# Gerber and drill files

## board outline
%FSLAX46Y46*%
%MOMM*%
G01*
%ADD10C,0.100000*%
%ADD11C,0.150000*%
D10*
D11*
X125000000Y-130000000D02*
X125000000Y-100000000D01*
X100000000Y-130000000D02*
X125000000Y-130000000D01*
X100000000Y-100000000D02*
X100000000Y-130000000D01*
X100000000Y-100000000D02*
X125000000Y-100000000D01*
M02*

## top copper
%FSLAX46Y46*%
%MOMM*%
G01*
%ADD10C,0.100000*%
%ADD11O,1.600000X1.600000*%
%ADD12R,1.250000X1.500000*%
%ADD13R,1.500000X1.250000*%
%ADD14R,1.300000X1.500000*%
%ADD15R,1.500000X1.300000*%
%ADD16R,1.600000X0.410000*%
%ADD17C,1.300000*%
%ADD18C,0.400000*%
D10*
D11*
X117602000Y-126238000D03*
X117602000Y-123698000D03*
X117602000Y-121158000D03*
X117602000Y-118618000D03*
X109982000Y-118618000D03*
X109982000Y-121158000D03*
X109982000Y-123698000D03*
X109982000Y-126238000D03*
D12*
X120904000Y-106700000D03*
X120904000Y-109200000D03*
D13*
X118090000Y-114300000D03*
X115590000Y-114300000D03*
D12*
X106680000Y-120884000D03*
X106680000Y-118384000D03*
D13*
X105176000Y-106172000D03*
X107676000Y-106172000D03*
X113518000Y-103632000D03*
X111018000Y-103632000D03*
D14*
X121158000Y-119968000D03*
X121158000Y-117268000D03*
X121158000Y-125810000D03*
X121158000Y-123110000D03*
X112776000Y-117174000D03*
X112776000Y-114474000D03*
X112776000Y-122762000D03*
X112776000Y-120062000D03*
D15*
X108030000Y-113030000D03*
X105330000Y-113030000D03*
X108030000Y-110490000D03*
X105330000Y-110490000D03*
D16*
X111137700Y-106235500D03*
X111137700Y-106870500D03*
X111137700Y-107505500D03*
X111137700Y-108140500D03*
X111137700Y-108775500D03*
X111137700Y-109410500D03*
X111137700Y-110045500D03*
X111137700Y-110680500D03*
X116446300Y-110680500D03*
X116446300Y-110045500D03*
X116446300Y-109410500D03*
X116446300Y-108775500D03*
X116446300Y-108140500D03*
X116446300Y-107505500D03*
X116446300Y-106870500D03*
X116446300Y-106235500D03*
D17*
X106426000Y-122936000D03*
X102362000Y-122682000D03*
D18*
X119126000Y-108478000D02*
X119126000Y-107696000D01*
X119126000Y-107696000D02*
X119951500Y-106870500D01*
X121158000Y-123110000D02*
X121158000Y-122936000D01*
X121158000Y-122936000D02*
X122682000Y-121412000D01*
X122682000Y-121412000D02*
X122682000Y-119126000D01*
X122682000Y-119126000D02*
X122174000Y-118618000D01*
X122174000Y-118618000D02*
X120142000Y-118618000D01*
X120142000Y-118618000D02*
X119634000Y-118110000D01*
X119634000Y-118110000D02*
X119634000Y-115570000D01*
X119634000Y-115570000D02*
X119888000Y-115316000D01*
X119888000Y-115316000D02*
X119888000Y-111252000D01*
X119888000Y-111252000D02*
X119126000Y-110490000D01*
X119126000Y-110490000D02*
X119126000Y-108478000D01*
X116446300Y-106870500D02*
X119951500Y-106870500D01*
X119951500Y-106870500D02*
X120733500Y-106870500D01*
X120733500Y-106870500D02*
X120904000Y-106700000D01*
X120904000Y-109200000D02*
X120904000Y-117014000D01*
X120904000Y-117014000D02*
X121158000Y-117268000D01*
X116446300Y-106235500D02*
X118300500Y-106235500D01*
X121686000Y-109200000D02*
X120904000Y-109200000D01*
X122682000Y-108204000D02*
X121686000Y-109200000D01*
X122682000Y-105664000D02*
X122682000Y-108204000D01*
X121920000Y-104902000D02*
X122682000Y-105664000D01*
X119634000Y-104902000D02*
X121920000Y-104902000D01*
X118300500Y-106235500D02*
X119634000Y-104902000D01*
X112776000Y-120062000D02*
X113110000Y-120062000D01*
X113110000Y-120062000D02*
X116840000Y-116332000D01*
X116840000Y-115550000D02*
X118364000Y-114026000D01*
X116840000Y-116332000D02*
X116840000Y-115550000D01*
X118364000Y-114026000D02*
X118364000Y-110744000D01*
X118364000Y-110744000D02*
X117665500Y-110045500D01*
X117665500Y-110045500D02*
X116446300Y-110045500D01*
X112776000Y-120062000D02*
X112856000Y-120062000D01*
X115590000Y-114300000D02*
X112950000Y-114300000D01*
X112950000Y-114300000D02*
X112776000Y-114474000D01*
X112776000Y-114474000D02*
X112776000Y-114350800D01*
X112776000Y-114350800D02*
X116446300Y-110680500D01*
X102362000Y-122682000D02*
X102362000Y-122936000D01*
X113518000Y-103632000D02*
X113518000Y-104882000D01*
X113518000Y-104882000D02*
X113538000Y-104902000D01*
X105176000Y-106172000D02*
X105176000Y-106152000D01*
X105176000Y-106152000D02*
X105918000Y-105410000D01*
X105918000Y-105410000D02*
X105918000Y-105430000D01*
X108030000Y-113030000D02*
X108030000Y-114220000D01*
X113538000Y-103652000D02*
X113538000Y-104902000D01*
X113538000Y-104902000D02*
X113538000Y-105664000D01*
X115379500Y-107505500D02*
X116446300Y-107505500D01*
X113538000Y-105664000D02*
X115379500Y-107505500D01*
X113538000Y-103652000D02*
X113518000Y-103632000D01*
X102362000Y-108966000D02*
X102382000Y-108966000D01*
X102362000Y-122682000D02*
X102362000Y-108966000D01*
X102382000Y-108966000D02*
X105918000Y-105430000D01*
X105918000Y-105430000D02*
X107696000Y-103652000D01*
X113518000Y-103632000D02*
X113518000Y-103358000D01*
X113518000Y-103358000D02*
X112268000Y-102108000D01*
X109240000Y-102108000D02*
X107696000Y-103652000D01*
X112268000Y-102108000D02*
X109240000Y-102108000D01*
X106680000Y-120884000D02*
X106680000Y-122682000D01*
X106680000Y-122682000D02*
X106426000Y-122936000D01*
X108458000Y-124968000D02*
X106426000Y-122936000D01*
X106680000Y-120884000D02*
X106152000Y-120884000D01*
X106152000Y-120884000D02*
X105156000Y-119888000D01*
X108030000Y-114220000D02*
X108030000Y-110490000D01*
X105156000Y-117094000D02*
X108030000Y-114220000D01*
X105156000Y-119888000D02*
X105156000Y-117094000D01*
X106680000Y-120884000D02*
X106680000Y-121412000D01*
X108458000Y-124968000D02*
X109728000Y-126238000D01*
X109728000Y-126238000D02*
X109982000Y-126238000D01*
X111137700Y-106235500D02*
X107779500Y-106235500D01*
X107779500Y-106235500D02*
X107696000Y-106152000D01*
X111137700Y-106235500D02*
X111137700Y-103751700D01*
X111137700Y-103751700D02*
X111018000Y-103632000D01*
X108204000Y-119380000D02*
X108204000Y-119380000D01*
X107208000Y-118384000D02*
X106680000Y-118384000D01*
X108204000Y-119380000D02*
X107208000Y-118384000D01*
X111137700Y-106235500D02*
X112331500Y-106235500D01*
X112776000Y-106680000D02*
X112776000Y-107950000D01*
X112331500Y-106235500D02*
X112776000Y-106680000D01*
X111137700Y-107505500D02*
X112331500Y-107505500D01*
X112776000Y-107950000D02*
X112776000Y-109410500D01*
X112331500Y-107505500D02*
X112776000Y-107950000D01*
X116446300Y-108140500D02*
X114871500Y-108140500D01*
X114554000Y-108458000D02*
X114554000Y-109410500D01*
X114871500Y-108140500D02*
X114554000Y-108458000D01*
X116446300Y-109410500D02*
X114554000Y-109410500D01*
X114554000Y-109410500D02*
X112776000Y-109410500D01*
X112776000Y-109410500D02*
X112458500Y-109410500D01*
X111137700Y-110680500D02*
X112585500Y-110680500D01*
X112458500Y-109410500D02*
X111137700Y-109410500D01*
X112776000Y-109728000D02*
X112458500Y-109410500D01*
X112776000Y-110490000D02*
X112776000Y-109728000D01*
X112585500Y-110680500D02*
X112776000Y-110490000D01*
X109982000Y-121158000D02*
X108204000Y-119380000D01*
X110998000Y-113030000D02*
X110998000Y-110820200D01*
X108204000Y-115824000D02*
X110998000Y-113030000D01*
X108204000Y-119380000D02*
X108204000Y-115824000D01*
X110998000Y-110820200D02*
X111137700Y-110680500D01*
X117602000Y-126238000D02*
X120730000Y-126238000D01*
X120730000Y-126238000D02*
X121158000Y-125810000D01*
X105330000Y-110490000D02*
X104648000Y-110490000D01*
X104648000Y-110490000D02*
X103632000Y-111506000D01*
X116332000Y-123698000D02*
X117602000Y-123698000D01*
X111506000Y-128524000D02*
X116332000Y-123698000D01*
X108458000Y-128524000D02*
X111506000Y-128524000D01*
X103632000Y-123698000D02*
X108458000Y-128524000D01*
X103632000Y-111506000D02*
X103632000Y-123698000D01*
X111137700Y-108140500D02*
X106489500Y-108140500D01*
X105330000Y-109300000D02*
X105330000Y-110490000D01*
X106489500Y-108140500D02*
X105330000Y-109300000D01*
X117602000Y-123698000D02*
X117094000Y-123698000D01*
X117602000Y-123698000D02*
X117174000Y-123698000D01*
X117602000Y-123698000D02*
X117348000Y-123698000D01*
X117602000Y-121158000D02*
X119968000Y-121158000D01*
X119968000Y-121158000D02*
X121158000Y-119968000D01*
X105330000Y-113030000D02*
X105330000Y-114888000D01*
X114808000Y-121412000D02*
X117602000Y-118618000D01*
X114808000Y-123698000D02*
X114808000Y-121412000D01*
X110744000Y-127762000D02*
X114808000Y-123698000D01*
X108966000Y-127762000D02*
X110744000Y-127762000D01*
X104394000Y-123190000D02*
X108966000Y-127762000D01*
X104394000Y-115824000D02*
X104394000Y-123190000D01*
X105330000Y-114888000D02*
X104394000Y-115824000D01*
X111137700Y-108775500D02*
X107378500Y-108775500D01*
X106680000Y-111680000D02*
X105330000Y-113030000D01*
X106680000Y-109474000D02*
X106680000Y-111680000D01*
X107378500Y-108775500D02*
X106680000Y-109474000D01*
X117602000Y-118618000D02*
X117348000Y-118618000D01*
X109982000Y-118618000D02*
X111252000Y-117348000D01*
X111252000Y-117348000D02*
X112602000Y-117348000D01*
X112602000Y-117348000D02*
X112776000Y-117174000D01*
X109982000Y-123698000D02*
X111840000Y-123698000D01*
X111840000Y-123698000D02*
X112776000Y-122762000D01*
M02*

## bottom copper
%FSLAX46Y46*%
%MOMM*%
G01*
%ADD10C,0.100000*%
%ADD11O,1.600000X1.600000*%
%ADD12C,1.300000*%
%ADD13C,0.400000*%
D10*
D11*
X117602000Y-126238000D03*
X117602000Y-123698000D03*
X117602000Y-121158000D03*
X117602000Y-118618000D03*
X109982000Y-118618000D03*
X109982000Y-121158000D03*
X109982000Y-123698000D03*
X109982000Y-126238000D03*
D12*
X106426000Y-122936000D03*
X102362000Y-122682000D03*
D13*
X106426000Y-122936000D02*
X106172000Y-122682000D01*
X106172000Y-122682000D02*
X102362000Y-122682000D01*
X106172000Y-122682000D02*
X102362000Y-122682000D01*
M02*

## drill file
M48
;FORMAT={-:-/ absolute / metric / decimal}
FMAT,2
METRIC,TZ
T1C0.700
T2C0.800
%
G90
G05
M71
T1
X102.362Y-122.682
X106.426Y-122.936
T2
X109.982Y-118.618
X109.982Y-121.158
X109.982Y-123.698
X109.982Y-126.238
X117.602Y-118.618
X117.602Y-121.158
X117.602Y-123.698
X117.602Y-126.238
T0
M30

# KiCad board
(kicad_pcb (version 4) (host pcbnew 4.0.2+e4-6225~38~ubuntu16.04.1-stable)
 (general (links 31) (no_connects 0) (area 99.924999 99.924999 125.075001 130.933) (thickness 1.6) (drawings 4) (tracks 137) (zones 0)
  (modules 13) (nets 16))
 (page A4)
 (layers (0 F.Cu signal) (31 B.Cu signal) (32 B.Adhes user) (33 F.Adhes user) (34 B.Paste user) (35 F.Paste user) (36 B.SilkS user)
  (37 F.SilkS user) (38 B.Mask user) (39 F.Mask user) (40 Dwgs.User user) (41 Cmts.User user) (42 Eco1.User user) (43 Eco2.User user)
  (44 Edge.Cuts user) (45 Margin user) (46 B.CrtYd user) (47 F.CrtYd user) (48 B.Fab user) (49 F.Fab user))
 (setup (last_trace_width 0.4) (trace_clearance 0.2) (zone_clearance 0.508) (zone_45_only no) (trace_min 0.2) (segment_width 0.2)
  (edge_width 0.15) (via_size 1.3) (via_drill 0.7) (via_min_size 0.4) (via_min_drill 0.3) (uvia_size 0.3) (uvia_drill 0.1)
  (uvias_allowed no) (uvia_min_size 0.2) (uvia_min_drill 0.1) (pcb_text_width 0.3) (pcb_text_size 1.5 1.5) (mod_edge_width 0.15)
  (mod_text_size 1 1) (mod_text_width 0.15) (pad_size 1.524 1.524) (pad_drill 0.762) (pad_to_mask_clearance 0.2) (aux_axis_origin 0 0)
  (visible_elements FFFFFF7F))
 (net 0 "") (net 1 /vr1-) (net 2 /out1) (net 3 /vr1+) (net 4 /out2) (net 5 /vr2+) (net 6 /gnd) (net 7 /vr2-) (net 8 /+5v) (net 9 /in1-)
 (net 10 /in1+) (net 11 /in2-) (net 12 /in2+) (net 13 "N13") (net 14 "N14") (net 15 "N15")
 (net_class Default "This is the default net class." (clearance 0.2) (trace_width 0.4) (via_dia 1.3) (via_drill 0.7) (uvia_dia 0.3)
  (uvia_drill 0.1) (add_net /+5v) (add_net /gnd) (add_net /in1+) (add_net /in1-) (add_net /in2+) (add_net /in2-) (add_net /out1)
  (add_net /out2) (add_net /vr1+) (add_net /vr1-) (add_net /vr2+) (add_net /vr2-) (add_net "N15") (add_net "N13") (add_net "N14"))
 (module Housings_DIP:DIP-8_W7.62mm (layer F.Cu) (at 117.602 126.238 180)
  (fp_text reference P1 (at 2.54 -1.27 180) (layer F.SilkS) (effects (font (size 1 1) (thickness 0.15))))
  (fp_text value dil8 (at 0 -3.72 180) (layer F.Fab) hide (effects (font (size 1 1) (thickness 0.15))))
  (pad 1 thru_hole oval (at 0 0 180) (size 1.6 1.6) (drill 0.8) (layers *.Cu *.Mask F.SilkS) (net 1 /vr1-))
  (pad 2 thru_hole oval (at 0 2.54 180) (size 1.6 1.6) (drill 0.8) (layers *.Cu *.Mask F.SilkS) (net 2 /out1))
  (pad 3 thru_hole oval (at 0 5.08 180) (size 1.6 1.6) (drill 0.8) (layers *.Cu *.Mask F.SilkS) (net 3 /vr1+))
  (pad 4 thru_hole oval (at 0 7.62 180) (size 1.6 1.6) (drill 0.8) (layers *.Cu *.Mask F.SilkS) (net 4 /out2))
  (pad 5 thru_hole oval (at 7.62 7.62 180) (size 1.6 1.6) (drill 0.8) (layers *.Cu *.Mask F.SilkS) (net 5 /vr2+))
  (pad 6 thru_hole oval (at 7.62 5.08 180) (size 1.6 1.6) (drill 0.8) (layers *.Cu *.Mask F.SilkS) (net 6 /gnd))
  (pad 7 thru_hole oval (at 7.62 2.54 180) (size 1.6 1.6) (drill 0.8) (layers *.Cu *.Mask F.SilkS) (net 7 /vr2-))
  (pad 8 thru_hole oval (at 7.62 0 180) (size 1.6 1.6) (drill 0.8) (layers *.Cu *.Mask F.SilkS) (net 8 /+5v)))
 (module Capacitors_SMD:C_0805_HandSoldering (layer F.Cu) (at 120.904 107.95 270)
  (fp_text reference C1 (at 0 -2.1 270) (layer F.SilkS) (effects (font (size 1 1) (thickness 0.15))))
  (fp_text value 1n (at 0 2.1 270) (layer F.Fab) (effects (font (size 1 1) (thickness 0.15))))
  (pad 1 smd rect (at -1.25 0 270) (size 1.5 1.25) (layers F.Cu F.Paste F.Mask) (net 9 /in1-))
  (pad 2 smd rect (at 1.25 0 270) (size 1.5 1.25) (layers F.Cu F.Paste F.Mask) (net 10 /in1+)))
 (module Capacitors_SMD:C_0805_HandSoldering (layer F.Cu) (at 116.84 114.3 180)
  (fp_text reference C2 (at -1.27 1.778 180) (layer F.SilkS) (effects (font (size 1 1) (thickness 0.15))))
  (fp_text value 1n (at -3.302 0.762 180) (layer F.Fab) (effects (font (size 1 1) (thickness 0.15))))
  (pad 1 smd rect (at -1.25 0 180) (size 1.5 1.25) (layers F.Cu F.Paste F.Mask) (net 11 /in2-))
  (pad 2 smd rect (at 1.25 0 180) (size 1.5 1.25) (layers F.Cu F.Paste F.Mask) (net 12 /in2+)))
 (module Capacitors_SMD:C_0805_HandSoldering (layer F.Cu) (at 106.68 119.634 90)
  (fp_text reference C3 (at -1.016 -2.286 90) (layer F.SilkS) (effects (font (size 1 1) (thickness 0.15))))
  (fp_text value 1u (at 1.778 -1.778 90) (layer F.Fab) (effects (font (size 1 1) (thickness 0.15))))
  (pad 1 smd rect (at -1.25 0 90) (size 1.5 1.25) (layers F.Cu F.Paste F.Mask) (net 8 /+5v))
  (pad 2 smd rect (at 1.25 0 90) (size 1.5 1.25) (layers F.Cu F.Paste F.Mask) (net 6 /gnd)))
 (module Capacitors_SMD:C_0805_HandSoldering (layer F.Cu) (at 106.426 106.172)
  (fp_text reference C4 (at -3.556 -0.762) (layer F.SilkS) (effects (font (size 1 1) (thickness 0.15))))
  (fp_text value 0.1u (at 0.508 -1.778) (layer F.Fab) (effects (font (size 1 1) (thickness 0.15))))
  (pad 1 smd rect (at -1.25 0) (size 1.5 1.25) (layers F.Cu F.Paste F.Mask) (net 8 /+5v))
  (pad 2 smd rect (at 1.25 0) (size 1.5 1.25) (layers F.Cu F.Paste F.Mask) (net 6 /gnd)))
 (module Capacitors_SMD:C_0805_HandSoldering (layer F.Cu) (at 112.268 103.632 180)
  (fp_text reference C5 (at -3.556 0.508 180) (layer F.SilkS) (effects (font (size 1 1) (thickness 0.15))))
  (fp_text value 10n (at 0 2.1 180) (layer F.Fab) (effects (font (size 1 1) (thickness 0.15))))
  (pad 1 smd rect (at -1.25 0 180) (size 1.5 1.25) (layers F.Cu F.Paste F.Mask) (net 8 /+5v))
  (pad 2 smd rect (at 1.25 0 180) (size 1.5 1.25) (layers F.Cu F.Paste F.Mask) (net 6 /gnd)))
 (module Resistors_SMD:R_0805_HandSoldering (layer F.Cu) (at 121.158 118.618 90)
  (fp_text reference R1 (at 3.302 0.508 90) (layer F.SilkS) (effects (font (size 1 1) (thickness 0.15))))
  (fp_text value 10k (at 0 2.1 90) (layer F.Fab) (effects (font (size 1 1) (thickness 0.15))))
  (pad 1 smd rect (at -1.35 0 90) (size 1.5 1.3) (layers F.Cu F.Paste F.Mask) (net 3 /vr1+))
  (pad 2 smd rect (at 1.35 0 90) (size 1.5 1.3) (layers F.Cu F.Paste F.Mask) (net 10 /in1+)))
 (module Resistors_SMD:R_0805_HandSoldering (layer F.Cu) (at 121.158 124.46 90)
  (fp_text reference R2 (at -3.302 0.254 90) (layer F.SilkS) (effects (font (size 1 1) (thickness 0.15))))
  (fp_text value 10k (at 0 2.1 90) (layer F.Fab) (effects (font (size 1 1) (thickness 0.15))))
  (pad 1 smd rect (at -1.35 0 90) (size 1.5 1.3) (layers F.Cu F.Paste F.Mask) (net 1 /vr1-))
  (pad 2 smd rect (at 1.35 0 90) (size 1.5 1.3) (layers F.Cu F.Paste F.Mask) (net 9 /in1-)))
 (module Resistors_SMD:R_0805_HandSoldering (layer F.Cu) (at 112.776 115.824 90)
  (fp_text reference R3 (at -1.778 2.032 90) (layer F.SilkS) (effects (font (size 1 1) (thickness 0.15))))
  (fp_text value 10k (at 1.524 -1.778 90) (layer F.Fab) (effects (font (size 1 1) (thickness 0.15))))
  (pad 1 smd rect (at -1.35 0 90) (size 1.5 1.3) (layers F.Cu F.Paste F.Mask) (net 5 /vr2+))
  (pad 2 smd rect (at 1.35 0 90) (size 1.5 1.3) (layers F.Cu F.Paste F.Mask) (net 12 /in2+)))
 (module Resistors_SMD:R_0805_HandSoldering (layer F.Cu) (at 112.776 121.412 90)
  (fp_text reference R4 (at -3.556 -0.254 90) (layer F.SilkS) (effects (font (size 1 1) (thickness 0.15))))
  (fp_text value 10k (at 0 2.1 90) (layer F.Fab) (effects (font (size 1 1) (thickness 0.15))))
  (pad 1 smd rect (at -1.35 0 90) (size 1.5 1.3) (layers F.Cu F.Paste F.Mask) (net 7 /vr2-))
  (pad 2 smd rect (at 1.35 0 90) (size 1.5 1.3) (layers F.Cu F.Paste F.Mask) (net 11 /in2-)))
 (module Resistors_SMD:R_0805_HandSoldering (layer F.Cu) (at 106.68 113.03 180)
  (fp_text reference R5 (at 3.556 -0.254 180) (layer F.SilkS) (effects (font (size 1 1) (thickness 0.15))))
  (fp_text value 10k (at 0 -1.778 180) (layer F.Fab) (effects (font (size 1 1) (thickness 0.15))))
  (pad 1 smd rect (at -1.35 0 180) (size 1.5 1.3) (layers F.Cu F.Paste F.Mask) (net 8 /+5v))
  (pad 2 smd rect (at 1.35 0 180) (size 1.5 1.3) (layers F.Cu F.Paste F.Mask) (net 4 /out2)))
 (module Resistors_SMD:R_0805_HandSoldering (layer F.Cu) (at 106.68 110.49 180)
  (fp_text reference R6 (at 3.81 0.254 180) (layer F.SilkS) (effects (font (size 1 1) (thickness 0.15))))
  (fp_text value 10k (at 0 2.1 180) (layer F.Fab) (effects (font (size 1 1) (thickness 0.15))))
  (pad 1 smd rect (at -1.35 0 180) (size 1.5 1.3) (layers F.Cu F.Paste F.Mask) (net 8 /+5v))
  (pad 2 smd rect (at 1.35 0 180) (size 1.5 1.3) (layers F.Cu F.Paste F.Mask) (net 2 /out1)))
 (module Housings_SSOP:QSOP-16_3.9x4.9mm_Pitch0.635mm (layer F.Cu) (at 113.792 108.458)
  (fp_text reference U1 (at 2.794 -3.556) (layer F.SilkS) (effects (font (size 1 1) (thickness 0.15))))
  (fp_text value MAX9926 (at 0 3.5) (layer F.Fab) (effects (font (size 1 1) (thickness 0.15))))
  (pad 1 smd rect (at -2.6543 -2.2225) (size 1.6 0.41) (layers F.Cu F.Paste F.Mask) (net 6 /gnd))
  (pad 2 smd rect (at -2.6543 -1.5875) (size 1.6 0.41) (layers F.Cu F.Paste F.Mask) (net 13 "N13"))
  (pad 3 smd rect (at -2.6543 -0.9525) (size 1.6 0.41) (layers F.Cu F.Paste F.Mask) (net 6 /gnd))
  (pad 4 smd rect (at -2.6543 -0.3175) (size 1.6 0.41) (layers F.Cu F.Paste F.Mask) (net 2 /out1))
  (pad 5 smd rect (at -2.6543 0.3175) (size 1.6 0.41) (layers F.Cu F.Paste F.Mask) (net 4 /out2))
  (pad 6 smd rect (at -2.6543 0.9525) (size 1.6 0.41) (layers F.Cu F.Paste F.Mask) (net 6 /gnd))
  (pad 7 smd rect (at -2.6543 1.5875) (size 1.6 0.41) (layers F.Cu F.Paste F.Mask) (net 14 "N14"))
  (pad 8 smd rect (at -2.6543 2.2225) (size 1.6 0.41) (layers F.Cu F.Paste F.Mask) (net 6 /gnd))
  (pad 9 smd rect (at 2.6543 2.2225) (size 1.6 0.41) (layers F.Cu F.Paste F.Mask) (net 12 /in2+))
  (pad 10 smd rect (at 2.6543 1.5875) (size 1.6 0.41) (layers F.Cu F.Paste F.Mask) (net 11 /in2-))
  (pad 11 smd rect (at 2.6543 0.9525) (size 1.6 0.41) (layers F.Cu F.Paste F.Mask) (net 6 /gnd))
  (pad 12 smd rect (at 2.6543 0.3175) (size 1.6 0.41) (layers F.Cu F.Paste F.Mask) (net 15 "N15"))
  (pad 13 smd rect (at 2.6543 -0.3175) (size 1.6 0.41) (layers F.Cu F.Paste F.Mask) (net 6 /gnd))
  (pad 14 smd rect (at 2.6543 -0.9525) (size 1.6 0.41) (layers F.Cu F.Paste F.Mask) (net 8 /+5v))
  (pad 15 smd rect (at 2.6543 -1.5875) (size 1.6 0.41) (layers F.Cu F.Paste F.Mask) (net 9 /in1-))
  (pad 16 smd rect (at 2.6543 -2.2225) (size 1.6 0.41) (layers F.Cu F.Paste F.Mask) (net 10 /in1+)))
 (gr_line (start 125 130) (end 125 100) (angle 90) (layer Edge.Cuts) (width 0.15))
 (gr_line (start 100 130) (end 125 130) (angle 90) (layer Edge.Cuts) (width 0.15))
 (gr_line (start 100 100) (end 100 130) (angle 90) (layer Edge.Cuts) (width 0.15))
 (gr_line (start 100 100) (end 125 100) (angle 90) (layer Edge.Cuts) (width 0.15))
 (segment (start 119.126 108.478) (end 119.126 107.696) (width 0.4) (layer F.Cu) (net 9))
 (segment (start 119.126 107.696) (end 119.9515 106.8705) (width 0.4) (layer F.Cu) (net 9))
 (segment (start 121.158 123.11) (end 121.158 122.936) (width 0.4) (layer F.Cu) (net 9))
 (segment (start 121.158 122.936) (end 122.682 121.412) (width 0.4) (layer F.Cu) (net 9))
 (segment (start 122.682 121.412) (end 122.682 119.126) (width 0.4) (layer F.Cu) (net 9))
 (segment (start 122.682 119.126) (end 122.174 118.618) (width 0.4) (layer F.Cu) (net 9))
 (segment (start 122.174 118.618) (end 120.142 118.618) (width 0.4) (layer F.Cu) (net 9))
 (segment (start 120.142 118.618) (end 119.634 118.11) (width 0.4) (layer F.Cu) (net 9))
 (segment (start 119.634 118.11) (end 119.634 115.57) (width 0.4) (layer F.Cu) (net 9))
 (segment (start 119.634 115.57) (end 119.888 115.316) (width 0.4) (layer F.Cu) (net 9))
 (segment (start 119.888 115.316) (end 119.888 111.252) (width 0.4) (layer F.Cu) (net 9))
 (segment (start 119.888 111.252) (end 119.126 110.49) (width 0.4) (layer F.Cu) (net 9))
 (segment (start 119.126 110.49) (end 119.126 108.478) (width 0.4) (layer F.Cu) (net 9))
 (segment (start 116.4463 106.8705) (end 119.9515 106.8705) (width 0.4) (layer F.Cu) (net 9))
 (segment (start 119.9515 106.8705) (end 120.7335 106.8705) (width 0.4) (layer F.Cu) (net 9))
 (segment (start 120.7335 106.8705) (end 120.904 106.7) (width 0.4) (layer F.Cu) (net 9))
 (segment (start 120.904 109.2) (end 120.904 117.014) (width 0.4) (layer F.Cu) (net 10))
 (segment (start 120.904 117.014) (end 121.158 117.268) (width 0.4) (layer F.Cu) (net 10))
 (segment (start 116.4463 106.2355) (end 118.3005 106.2355) (width 0.4) (layer F.Cu) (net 10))
 (segment (start 121.686 109.2) (end 120.904 109.2) (width 0.4) (layer F.Cu) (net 10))
 (segment (start 122.682 108.204) (end 121.686 109.2) (width 0.4) (layer F.Cu) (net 10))
 (segment (start 122.682 105.664) (end 122.682 108.204) (width 0.4) (layer F.Cu) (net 10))
 (segment (start 121.92 104.902) (end 122.682 105.664) (width 0.4) (layer F.Cu) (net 10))
 (segment (start 119.634 104.902) (end 121.92 104.902) (width 0.4) (layer F.Cu) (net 10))
 (segment (start 118.3005 106.2355) (end 119.634 104.902) (width 0.4) (layer F.Cu) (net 10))
 (segment (start 112.776 120.062) (end 113.11 120.062) (width 0.4) (layer F.Cu) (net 11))
 (segment (start 113.11 120.062) (end 116.84 116.332) (width 0.4) (layer F.Cu) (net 11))
 (segment (start 116.84 115.55) (end 118.364 114.026) (width 0.4) (layer F.Cu) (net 11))
 (segment (start 116.84 116.332) (end 116.84 115.55) (width 0.4) (layer F.Cu) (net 11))
 (segment (start 118.364 114.026) (end 118.364 110.744) (width 0.4) (layer F.Cu) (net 11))
 (segment (start 118.364 110.744) (end 117.6655 110.0455) (width 0.4) (layer F.Cu) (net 11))
 (segment (start 117.6655 110.0455) (end 116.4463 110.0455) (width 0.4) (layer F.Cu) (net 11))
 (segment (start 112.776 120.062) (end 112.856 120.062) (width 0.4) (layer F.Cu) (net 11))
 (segment (start 115.59 114.3) (end 112.95 114.3) (width 0.4) (layer F.Cu) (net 12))
 (segment (start 112.95 114.3) (end 112.776 114.474) (width 0.4) (layer F.Cu) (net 12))
 (segment (start 112.776 114.474) (end 112.776 114.3508) (width 0.4) (layer F.Cu) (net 12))
 (segment (start 112.776 114.3508) (end 116.4463 110.6805) (width 0.4) (layer F.Cu) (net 12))
 (via (at 106.426 122.936) (size 1.3) (drill 0.7) (layers F.Cu B.Cu) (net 8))
 (segment (start 106.426 122.936) (end 106.172 122.682) (width 0.4) (layer B.Cu) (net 8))
 (segment (start 106.172 122.682) (end 102.362 122.682) (width 0.4) (layer B.Cu) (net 8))
 (via (at 102.362 122.682) (size 1.3) (drill 0.7) (layers F.Cu B.Cu) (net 8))
 (segment (start 102.362 122.682) (end 102.362 122.936) (width 0.4) (layer F.Cu) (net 8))
 (segment (start 113.518 103.632) (end 113.518 104.882) (width 0.4) (layer F.Cu) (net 8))
 (segment (start 113.518 104.882) (end 113.538 104.902) (width 0.4) (layer F.Cu) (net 8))
 (segment (start 105.176 106.172) (end 105.176 106.152) (width 0.4) (layer F.Cu) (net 8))
 (segment (start 105.176 106.152) (end 105.918 105.41) (width 0.4) (layer F.Cu) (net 8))
 (segment (start 105.918 105.41) (end 105.918 105.43) (width 0.4) (layer F.Cu) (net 8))
 (segment (start 108.03 113.03) (end 108.03 114.22) (width 0.4) (layer F.Cu) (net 8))
 (segment (start 113.538 103.652) (end 113.538 104.902) (width 0.4) (layer F.Cu) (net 8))
 (segment (start 113.538 104.902) (end 113.538 105.664) (width 0.4) (layer F.Cu) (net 8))
 (segment (start 115.3795 107.5055) (end 116.4463 107.5055) (width 0.4) (layer F.Cu) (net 8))
 (segment (start 113.538 105.664) (end 115.3795 107.5055) (width 0.4) (layer F.Cu) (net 8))
 (segment (start 113.538 103.652) (end 113.518 103.632) (width 0.4) (layer F.Cu) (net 8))
 (segment (start 102.362 108.966) (end 102.382 108.966) (width 0.4) (layer F.Cu) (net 8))
 (segment (start 102.362 122.682) (end 102.362 108.966) (width 0.4) (layer F.Cu) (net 8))
 (segment (start 106.172 122.682) (end 102.362 122.682) (width 0.4) (layer B.Cu) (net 8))
 (segment (start 102.382 108.966) (end 105.918 105.43) (width 0.4) (layer F.Cu) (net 8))
 (segment (start 105.918 105.43) (end 107.696 103.652) (width 0.4) (layer F.Cu) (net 8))
 (segment (start 113.518 103.632) (end 113.518 103.358) (width 0.4) (layer F.Cu) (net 8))
 (segment (start 113.518 103.358) (end 112.268 102.108) (width 0.4) (layer F.Cu) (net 8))
 (segment (start 109.24 102.108) (end 107.696 103.652) (width 0.4) (layer F.Cu) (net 8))
 (segment (start 112.268 102.108) (end 109.24 102.108) (width 0.4) (layer F.Cu) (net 8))
 (segment (start 106.68 120.884) (end 106.68 122.682) (width 0.4) (layer F.Cu) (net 8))
 (segment (start 106.68 122.682) (end 106.426 122.936) (width 0.4) (layer F.Cu) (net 8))
 (segment (start 108.458 124.968) (end 106.426 122.936) (width 0.4) (layer F.Cu) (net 8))
 (segment (start 106.68 120.884) (end 106.152 120.884) (width 0.4) (layer F.Cu) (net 8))
 (segment (start 106.152 120.884) (end 105.156 119.888) (width 0.4) (layer F.Cu) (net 8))
 (segment (start 108.03 114.22) (end 108.03 110.49) (width 0.4) (layer F.Cu) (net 8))
 (segment (start 105.156 117.094) (end 108.03 114.22) (width 0.4) (layer F.Cu) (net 8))
 (segment (start 105.156 119.888) (end 105.156 117.094) (width 0.4) (layer F.Cu) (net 8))
 (segment (start 106.68 120.884) (end 106.68 121.412) (width 0.4) (layer F.Cu) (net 8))
 (segment (start 108.458 124.968) (end 109.728 126.238) (width 0.4) (layer F.Cu) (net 8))
 (segment (start 109.728 126.238) (end 109.982 126.238) (width 0.4) (layer F.Cu) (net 8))
 (segment (start 111.1377 106.2355) (end 107.7795 106.2355) (width 0.4) (layer F.Cu) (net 6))
 (segment (start 107.7795 106.2355) (end 107.696 106.152) (width 0.4) (layer F.Cu) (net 6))
 (segment (start 111.1377 106.2355) (end 111.1377 103.7517) (width 0.4) (layer F.Cu) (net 6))
 (segment (start 111.1377 103.7517) (end 111.018 103.632) (width 0.4) (layer F.Cu) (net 6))
 (segment (start 108.204 119.38) (end 108.204 119.38) (width 0.4) (layer F.Cu) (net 6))
 (segment (start 107.208 118.384) (end 106.68 118.384) (width 0.4) (layer F.Cu) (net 6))
 (segment (start 108.204 119.38) (end 107.208 118.384) (width 0.4) (layer F.Cu) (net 6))
 (segment (start 111.1377 106.2355) (end 112.3315 106.2355) (width 0.4) (layer F.Cu) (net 6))
 (segment (start 112.776 106.68) (end 112.776 107.95) (width 0.4) (layer F.Cu) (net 6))
 (segment (start 112.3315 106.2355) (end 112.776 106.68) (width 0.4) (layer F.Cu) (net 6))
 (segment (start 111.1377 107.5055) (end 112.3315 107.5055) (width 0.4) (layer F.Cu) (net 6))
 (segment (start 112.776 107.95) (end 112.776 109.4105) (width 0.4) (layer F.Cu) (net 6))
 (segment (start 112.3315 107.5055) (end 112.776 107.95) (width 0.4) (layer F.Cu) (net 6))
 (segment (start 116.4463 108.1405) (end 114.8715 108.1405) (width 0.4) (layer F.Cu) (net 6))
 (segment (start 114.554 108.458) (end 114.554 109.4105) (width 0.4) (layer F.Cu) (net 6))
 (segment (start 114.8715 108.1405) (end 114.554 108.458) (width 0.4) (layer F.Cu) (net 6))
 (segment (start 116.4463 109.4105) (end 114.554 109.4105) (width 0.4) (layer F.Cu) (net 6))
 (segment (start 114.554 109.4105) (end 112.776 109.4105) (width 0.4) (layer F.Cu) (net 6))
 (segment (start 112.776 109.4105) (end 112.4585 109.4105) (width 0.4) (layer F.Cu) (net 6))
 (segment (start 111.1377 110.6805) (end 112.5855 110.6805) (width 0.4) (layer F.Cu) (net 6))
 (segment (start 112.4585 109.4105) (end 111.1377 109.4105) (width 0.4) (layer F.Cu) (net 6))
 (segment (start 112.776 109.728) (end 112.4585 109.4105) (width 0.4) (layer F.Cu) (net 6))
 (segment (start 112.776 110.49) (end 112.776 109.728) (width 0.4) (layer F.Cu) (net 6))
 (segment (start 112.5855 110.6805) (end 112.776 110.49) (width 0.4) (layer F.Cu) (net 6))
 (segment (start 109.982 121.158) (end 108.204 119.38) (width 0.4) (layer F.Cu) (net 6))
 (segment (start 110.998 113.03) (end 110.998 110.8202) (width 0.4) (layer F.Cu) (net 6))
 (segment (start 108.204 115.824) (end 110.998 113.03) (width 0.4) (layer F.Cu) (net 6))
 (segment (start 108.204 119.38) (end 108.204 115.824) (width 0.4) (layer F.Cu) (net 6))
 (segment (start 110.998 110.8202) (end 111.1377 110.6805) (width 0.4) (layer F.Cu) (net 6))
 (segment (start 117.602 126.238) (end 120.73 126.238) (width 0.4) (layer F.Cu) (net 1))
 (segment (start 120.73 126.238) (end 121.158 125.81) (width 0.4) (layer F.Cu) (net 1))
 (segment (start 105.33 110.49) (end 104.648 110.49) (width 0.4) (layer F.Cu) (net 2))
 (segment (start 104.648 110.49) (end 103.632 111.506) (width 0.4) (layer F.Cu) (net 2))
 (segment (start 116.332 123.698) (end 117.602 123.698) (width 0.4) (layer F.Cu) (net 2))
 (segment (start 111.506 128.524) (end 116.332 123.698) (width 0.4) (layer F.Cu) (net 2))
 (segment (start 108.458 128.524) (end 111.506 128.524) (width 0.4) (layer F.Cu) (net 2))
 (segment (start 103.632 123.698) (end 108.458 128.524) (width 0.4) (layer F.Cu) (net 2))
 (segment (start 103.632 111.506) (end 103.632 123.698) (width 0.4) (layer F.Cu) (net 2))
 (segment (start 111.1377 108.1405) (end 106.4895 108.1405) (width 0.4) (layer F.Cu) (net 2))
 (segment (start 105.33 109.3) (end 105.33 110.49) (width 0.4) (layer F.Cu) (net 2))
 (segment (start 106.4895 108.1405) (end 105.33 109.3) (width 0.4) (layer F.Cu) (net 2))
 (segment (start 117.602 123.698) (end 117.094 123.698) (width 0.4) (layer F.Cu) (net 2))
 (segment (start 117.602 123.698) (end 117.174 123.698) (width 0.4) (layer F.Cu) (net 2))
 (segment (start 117.602 123.698) (end 117.348 123.698) (width 0.4) (layer F.Cu) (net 2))
 (segment (start 117.602 121.158) (end 119.968 121.158) (width 0.4) (layer F.Cu) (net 3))
 (segment (start 119.968 121.158) (end 121.158 119.968) (width 0.4) (layer F.Cu) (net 3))
 (segment (start 105.33 113.03) (end 105.33 114.888) (width 0.4) (layer F.Cu) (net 4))
 (segment (start 114.808 121.412) (end 117.602 118.618) (width 0.4) (layer F.Cu) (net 4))
 (segment (start 114.808 123.698) (end 114.808 121.412) (width 0.4) (layer F.Cu) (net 4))
 (segment (start 110.744 127.762) (end 114.808 123.698) (width 0.4) (layer F.Cu) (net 4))
 (segment (start 108.966 127.762) (end 110.744 127.762) (width 0.4) (layer F.Cu) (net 4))
 (segment (start 104.394 123.19) (end 108.966 127.762) (width 0.4) (layer F.Cu) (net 4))
 (segment (start 104.394 115.824) (end 104.394 123.19) (width 0.4) (layer F.Cu) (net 4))
 (segment (start 105.33 114.888) (end 104.394 115.824) (width 0.4) (layer F.Cu) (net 4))
 (segment (start 111.1377 108.7755) (end 107.3785 108.7755) (width 0.4) (layer F.Cu) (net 4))
 (segment (start 106.68 111.68) (end 105.33 113.03) (width 0.4) (layer F.Cu) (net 4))
 (segment (start 106.68 109.474) (end 106.68 111.68) (width 0.4) (layer F.Cu) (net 4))
 (segment (start 107.3785 108.7755) (end 106.68 109.474) (width 0.4) (layer F.Cu) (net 4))
 (segment (start 117.602 118.618) (end 117.348 118.618) (width 0.4) (layer F.Cu) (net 4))
 (segment (start 109.982 118.618) (end 111.252 117.348) (width 0.4) (layer F.Cu) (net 5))
 (segment (start 111.252 117.348) (end 112.602 117.348) (width 0.4) (layer F.Cu) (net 5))
 (segment (start 112.602 117.348) (end 112.776 117.174) (width 0.4) (layer F.Cu) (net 5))
 (segment (start 109.982 123.698) (end 111.84 123.698) (width 0.4) (layer F.Cu) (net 7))
 (segment (start 111.84 123.698) (end 112.776 122.762) (width 0.4) (layer F.Cu) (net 7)))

